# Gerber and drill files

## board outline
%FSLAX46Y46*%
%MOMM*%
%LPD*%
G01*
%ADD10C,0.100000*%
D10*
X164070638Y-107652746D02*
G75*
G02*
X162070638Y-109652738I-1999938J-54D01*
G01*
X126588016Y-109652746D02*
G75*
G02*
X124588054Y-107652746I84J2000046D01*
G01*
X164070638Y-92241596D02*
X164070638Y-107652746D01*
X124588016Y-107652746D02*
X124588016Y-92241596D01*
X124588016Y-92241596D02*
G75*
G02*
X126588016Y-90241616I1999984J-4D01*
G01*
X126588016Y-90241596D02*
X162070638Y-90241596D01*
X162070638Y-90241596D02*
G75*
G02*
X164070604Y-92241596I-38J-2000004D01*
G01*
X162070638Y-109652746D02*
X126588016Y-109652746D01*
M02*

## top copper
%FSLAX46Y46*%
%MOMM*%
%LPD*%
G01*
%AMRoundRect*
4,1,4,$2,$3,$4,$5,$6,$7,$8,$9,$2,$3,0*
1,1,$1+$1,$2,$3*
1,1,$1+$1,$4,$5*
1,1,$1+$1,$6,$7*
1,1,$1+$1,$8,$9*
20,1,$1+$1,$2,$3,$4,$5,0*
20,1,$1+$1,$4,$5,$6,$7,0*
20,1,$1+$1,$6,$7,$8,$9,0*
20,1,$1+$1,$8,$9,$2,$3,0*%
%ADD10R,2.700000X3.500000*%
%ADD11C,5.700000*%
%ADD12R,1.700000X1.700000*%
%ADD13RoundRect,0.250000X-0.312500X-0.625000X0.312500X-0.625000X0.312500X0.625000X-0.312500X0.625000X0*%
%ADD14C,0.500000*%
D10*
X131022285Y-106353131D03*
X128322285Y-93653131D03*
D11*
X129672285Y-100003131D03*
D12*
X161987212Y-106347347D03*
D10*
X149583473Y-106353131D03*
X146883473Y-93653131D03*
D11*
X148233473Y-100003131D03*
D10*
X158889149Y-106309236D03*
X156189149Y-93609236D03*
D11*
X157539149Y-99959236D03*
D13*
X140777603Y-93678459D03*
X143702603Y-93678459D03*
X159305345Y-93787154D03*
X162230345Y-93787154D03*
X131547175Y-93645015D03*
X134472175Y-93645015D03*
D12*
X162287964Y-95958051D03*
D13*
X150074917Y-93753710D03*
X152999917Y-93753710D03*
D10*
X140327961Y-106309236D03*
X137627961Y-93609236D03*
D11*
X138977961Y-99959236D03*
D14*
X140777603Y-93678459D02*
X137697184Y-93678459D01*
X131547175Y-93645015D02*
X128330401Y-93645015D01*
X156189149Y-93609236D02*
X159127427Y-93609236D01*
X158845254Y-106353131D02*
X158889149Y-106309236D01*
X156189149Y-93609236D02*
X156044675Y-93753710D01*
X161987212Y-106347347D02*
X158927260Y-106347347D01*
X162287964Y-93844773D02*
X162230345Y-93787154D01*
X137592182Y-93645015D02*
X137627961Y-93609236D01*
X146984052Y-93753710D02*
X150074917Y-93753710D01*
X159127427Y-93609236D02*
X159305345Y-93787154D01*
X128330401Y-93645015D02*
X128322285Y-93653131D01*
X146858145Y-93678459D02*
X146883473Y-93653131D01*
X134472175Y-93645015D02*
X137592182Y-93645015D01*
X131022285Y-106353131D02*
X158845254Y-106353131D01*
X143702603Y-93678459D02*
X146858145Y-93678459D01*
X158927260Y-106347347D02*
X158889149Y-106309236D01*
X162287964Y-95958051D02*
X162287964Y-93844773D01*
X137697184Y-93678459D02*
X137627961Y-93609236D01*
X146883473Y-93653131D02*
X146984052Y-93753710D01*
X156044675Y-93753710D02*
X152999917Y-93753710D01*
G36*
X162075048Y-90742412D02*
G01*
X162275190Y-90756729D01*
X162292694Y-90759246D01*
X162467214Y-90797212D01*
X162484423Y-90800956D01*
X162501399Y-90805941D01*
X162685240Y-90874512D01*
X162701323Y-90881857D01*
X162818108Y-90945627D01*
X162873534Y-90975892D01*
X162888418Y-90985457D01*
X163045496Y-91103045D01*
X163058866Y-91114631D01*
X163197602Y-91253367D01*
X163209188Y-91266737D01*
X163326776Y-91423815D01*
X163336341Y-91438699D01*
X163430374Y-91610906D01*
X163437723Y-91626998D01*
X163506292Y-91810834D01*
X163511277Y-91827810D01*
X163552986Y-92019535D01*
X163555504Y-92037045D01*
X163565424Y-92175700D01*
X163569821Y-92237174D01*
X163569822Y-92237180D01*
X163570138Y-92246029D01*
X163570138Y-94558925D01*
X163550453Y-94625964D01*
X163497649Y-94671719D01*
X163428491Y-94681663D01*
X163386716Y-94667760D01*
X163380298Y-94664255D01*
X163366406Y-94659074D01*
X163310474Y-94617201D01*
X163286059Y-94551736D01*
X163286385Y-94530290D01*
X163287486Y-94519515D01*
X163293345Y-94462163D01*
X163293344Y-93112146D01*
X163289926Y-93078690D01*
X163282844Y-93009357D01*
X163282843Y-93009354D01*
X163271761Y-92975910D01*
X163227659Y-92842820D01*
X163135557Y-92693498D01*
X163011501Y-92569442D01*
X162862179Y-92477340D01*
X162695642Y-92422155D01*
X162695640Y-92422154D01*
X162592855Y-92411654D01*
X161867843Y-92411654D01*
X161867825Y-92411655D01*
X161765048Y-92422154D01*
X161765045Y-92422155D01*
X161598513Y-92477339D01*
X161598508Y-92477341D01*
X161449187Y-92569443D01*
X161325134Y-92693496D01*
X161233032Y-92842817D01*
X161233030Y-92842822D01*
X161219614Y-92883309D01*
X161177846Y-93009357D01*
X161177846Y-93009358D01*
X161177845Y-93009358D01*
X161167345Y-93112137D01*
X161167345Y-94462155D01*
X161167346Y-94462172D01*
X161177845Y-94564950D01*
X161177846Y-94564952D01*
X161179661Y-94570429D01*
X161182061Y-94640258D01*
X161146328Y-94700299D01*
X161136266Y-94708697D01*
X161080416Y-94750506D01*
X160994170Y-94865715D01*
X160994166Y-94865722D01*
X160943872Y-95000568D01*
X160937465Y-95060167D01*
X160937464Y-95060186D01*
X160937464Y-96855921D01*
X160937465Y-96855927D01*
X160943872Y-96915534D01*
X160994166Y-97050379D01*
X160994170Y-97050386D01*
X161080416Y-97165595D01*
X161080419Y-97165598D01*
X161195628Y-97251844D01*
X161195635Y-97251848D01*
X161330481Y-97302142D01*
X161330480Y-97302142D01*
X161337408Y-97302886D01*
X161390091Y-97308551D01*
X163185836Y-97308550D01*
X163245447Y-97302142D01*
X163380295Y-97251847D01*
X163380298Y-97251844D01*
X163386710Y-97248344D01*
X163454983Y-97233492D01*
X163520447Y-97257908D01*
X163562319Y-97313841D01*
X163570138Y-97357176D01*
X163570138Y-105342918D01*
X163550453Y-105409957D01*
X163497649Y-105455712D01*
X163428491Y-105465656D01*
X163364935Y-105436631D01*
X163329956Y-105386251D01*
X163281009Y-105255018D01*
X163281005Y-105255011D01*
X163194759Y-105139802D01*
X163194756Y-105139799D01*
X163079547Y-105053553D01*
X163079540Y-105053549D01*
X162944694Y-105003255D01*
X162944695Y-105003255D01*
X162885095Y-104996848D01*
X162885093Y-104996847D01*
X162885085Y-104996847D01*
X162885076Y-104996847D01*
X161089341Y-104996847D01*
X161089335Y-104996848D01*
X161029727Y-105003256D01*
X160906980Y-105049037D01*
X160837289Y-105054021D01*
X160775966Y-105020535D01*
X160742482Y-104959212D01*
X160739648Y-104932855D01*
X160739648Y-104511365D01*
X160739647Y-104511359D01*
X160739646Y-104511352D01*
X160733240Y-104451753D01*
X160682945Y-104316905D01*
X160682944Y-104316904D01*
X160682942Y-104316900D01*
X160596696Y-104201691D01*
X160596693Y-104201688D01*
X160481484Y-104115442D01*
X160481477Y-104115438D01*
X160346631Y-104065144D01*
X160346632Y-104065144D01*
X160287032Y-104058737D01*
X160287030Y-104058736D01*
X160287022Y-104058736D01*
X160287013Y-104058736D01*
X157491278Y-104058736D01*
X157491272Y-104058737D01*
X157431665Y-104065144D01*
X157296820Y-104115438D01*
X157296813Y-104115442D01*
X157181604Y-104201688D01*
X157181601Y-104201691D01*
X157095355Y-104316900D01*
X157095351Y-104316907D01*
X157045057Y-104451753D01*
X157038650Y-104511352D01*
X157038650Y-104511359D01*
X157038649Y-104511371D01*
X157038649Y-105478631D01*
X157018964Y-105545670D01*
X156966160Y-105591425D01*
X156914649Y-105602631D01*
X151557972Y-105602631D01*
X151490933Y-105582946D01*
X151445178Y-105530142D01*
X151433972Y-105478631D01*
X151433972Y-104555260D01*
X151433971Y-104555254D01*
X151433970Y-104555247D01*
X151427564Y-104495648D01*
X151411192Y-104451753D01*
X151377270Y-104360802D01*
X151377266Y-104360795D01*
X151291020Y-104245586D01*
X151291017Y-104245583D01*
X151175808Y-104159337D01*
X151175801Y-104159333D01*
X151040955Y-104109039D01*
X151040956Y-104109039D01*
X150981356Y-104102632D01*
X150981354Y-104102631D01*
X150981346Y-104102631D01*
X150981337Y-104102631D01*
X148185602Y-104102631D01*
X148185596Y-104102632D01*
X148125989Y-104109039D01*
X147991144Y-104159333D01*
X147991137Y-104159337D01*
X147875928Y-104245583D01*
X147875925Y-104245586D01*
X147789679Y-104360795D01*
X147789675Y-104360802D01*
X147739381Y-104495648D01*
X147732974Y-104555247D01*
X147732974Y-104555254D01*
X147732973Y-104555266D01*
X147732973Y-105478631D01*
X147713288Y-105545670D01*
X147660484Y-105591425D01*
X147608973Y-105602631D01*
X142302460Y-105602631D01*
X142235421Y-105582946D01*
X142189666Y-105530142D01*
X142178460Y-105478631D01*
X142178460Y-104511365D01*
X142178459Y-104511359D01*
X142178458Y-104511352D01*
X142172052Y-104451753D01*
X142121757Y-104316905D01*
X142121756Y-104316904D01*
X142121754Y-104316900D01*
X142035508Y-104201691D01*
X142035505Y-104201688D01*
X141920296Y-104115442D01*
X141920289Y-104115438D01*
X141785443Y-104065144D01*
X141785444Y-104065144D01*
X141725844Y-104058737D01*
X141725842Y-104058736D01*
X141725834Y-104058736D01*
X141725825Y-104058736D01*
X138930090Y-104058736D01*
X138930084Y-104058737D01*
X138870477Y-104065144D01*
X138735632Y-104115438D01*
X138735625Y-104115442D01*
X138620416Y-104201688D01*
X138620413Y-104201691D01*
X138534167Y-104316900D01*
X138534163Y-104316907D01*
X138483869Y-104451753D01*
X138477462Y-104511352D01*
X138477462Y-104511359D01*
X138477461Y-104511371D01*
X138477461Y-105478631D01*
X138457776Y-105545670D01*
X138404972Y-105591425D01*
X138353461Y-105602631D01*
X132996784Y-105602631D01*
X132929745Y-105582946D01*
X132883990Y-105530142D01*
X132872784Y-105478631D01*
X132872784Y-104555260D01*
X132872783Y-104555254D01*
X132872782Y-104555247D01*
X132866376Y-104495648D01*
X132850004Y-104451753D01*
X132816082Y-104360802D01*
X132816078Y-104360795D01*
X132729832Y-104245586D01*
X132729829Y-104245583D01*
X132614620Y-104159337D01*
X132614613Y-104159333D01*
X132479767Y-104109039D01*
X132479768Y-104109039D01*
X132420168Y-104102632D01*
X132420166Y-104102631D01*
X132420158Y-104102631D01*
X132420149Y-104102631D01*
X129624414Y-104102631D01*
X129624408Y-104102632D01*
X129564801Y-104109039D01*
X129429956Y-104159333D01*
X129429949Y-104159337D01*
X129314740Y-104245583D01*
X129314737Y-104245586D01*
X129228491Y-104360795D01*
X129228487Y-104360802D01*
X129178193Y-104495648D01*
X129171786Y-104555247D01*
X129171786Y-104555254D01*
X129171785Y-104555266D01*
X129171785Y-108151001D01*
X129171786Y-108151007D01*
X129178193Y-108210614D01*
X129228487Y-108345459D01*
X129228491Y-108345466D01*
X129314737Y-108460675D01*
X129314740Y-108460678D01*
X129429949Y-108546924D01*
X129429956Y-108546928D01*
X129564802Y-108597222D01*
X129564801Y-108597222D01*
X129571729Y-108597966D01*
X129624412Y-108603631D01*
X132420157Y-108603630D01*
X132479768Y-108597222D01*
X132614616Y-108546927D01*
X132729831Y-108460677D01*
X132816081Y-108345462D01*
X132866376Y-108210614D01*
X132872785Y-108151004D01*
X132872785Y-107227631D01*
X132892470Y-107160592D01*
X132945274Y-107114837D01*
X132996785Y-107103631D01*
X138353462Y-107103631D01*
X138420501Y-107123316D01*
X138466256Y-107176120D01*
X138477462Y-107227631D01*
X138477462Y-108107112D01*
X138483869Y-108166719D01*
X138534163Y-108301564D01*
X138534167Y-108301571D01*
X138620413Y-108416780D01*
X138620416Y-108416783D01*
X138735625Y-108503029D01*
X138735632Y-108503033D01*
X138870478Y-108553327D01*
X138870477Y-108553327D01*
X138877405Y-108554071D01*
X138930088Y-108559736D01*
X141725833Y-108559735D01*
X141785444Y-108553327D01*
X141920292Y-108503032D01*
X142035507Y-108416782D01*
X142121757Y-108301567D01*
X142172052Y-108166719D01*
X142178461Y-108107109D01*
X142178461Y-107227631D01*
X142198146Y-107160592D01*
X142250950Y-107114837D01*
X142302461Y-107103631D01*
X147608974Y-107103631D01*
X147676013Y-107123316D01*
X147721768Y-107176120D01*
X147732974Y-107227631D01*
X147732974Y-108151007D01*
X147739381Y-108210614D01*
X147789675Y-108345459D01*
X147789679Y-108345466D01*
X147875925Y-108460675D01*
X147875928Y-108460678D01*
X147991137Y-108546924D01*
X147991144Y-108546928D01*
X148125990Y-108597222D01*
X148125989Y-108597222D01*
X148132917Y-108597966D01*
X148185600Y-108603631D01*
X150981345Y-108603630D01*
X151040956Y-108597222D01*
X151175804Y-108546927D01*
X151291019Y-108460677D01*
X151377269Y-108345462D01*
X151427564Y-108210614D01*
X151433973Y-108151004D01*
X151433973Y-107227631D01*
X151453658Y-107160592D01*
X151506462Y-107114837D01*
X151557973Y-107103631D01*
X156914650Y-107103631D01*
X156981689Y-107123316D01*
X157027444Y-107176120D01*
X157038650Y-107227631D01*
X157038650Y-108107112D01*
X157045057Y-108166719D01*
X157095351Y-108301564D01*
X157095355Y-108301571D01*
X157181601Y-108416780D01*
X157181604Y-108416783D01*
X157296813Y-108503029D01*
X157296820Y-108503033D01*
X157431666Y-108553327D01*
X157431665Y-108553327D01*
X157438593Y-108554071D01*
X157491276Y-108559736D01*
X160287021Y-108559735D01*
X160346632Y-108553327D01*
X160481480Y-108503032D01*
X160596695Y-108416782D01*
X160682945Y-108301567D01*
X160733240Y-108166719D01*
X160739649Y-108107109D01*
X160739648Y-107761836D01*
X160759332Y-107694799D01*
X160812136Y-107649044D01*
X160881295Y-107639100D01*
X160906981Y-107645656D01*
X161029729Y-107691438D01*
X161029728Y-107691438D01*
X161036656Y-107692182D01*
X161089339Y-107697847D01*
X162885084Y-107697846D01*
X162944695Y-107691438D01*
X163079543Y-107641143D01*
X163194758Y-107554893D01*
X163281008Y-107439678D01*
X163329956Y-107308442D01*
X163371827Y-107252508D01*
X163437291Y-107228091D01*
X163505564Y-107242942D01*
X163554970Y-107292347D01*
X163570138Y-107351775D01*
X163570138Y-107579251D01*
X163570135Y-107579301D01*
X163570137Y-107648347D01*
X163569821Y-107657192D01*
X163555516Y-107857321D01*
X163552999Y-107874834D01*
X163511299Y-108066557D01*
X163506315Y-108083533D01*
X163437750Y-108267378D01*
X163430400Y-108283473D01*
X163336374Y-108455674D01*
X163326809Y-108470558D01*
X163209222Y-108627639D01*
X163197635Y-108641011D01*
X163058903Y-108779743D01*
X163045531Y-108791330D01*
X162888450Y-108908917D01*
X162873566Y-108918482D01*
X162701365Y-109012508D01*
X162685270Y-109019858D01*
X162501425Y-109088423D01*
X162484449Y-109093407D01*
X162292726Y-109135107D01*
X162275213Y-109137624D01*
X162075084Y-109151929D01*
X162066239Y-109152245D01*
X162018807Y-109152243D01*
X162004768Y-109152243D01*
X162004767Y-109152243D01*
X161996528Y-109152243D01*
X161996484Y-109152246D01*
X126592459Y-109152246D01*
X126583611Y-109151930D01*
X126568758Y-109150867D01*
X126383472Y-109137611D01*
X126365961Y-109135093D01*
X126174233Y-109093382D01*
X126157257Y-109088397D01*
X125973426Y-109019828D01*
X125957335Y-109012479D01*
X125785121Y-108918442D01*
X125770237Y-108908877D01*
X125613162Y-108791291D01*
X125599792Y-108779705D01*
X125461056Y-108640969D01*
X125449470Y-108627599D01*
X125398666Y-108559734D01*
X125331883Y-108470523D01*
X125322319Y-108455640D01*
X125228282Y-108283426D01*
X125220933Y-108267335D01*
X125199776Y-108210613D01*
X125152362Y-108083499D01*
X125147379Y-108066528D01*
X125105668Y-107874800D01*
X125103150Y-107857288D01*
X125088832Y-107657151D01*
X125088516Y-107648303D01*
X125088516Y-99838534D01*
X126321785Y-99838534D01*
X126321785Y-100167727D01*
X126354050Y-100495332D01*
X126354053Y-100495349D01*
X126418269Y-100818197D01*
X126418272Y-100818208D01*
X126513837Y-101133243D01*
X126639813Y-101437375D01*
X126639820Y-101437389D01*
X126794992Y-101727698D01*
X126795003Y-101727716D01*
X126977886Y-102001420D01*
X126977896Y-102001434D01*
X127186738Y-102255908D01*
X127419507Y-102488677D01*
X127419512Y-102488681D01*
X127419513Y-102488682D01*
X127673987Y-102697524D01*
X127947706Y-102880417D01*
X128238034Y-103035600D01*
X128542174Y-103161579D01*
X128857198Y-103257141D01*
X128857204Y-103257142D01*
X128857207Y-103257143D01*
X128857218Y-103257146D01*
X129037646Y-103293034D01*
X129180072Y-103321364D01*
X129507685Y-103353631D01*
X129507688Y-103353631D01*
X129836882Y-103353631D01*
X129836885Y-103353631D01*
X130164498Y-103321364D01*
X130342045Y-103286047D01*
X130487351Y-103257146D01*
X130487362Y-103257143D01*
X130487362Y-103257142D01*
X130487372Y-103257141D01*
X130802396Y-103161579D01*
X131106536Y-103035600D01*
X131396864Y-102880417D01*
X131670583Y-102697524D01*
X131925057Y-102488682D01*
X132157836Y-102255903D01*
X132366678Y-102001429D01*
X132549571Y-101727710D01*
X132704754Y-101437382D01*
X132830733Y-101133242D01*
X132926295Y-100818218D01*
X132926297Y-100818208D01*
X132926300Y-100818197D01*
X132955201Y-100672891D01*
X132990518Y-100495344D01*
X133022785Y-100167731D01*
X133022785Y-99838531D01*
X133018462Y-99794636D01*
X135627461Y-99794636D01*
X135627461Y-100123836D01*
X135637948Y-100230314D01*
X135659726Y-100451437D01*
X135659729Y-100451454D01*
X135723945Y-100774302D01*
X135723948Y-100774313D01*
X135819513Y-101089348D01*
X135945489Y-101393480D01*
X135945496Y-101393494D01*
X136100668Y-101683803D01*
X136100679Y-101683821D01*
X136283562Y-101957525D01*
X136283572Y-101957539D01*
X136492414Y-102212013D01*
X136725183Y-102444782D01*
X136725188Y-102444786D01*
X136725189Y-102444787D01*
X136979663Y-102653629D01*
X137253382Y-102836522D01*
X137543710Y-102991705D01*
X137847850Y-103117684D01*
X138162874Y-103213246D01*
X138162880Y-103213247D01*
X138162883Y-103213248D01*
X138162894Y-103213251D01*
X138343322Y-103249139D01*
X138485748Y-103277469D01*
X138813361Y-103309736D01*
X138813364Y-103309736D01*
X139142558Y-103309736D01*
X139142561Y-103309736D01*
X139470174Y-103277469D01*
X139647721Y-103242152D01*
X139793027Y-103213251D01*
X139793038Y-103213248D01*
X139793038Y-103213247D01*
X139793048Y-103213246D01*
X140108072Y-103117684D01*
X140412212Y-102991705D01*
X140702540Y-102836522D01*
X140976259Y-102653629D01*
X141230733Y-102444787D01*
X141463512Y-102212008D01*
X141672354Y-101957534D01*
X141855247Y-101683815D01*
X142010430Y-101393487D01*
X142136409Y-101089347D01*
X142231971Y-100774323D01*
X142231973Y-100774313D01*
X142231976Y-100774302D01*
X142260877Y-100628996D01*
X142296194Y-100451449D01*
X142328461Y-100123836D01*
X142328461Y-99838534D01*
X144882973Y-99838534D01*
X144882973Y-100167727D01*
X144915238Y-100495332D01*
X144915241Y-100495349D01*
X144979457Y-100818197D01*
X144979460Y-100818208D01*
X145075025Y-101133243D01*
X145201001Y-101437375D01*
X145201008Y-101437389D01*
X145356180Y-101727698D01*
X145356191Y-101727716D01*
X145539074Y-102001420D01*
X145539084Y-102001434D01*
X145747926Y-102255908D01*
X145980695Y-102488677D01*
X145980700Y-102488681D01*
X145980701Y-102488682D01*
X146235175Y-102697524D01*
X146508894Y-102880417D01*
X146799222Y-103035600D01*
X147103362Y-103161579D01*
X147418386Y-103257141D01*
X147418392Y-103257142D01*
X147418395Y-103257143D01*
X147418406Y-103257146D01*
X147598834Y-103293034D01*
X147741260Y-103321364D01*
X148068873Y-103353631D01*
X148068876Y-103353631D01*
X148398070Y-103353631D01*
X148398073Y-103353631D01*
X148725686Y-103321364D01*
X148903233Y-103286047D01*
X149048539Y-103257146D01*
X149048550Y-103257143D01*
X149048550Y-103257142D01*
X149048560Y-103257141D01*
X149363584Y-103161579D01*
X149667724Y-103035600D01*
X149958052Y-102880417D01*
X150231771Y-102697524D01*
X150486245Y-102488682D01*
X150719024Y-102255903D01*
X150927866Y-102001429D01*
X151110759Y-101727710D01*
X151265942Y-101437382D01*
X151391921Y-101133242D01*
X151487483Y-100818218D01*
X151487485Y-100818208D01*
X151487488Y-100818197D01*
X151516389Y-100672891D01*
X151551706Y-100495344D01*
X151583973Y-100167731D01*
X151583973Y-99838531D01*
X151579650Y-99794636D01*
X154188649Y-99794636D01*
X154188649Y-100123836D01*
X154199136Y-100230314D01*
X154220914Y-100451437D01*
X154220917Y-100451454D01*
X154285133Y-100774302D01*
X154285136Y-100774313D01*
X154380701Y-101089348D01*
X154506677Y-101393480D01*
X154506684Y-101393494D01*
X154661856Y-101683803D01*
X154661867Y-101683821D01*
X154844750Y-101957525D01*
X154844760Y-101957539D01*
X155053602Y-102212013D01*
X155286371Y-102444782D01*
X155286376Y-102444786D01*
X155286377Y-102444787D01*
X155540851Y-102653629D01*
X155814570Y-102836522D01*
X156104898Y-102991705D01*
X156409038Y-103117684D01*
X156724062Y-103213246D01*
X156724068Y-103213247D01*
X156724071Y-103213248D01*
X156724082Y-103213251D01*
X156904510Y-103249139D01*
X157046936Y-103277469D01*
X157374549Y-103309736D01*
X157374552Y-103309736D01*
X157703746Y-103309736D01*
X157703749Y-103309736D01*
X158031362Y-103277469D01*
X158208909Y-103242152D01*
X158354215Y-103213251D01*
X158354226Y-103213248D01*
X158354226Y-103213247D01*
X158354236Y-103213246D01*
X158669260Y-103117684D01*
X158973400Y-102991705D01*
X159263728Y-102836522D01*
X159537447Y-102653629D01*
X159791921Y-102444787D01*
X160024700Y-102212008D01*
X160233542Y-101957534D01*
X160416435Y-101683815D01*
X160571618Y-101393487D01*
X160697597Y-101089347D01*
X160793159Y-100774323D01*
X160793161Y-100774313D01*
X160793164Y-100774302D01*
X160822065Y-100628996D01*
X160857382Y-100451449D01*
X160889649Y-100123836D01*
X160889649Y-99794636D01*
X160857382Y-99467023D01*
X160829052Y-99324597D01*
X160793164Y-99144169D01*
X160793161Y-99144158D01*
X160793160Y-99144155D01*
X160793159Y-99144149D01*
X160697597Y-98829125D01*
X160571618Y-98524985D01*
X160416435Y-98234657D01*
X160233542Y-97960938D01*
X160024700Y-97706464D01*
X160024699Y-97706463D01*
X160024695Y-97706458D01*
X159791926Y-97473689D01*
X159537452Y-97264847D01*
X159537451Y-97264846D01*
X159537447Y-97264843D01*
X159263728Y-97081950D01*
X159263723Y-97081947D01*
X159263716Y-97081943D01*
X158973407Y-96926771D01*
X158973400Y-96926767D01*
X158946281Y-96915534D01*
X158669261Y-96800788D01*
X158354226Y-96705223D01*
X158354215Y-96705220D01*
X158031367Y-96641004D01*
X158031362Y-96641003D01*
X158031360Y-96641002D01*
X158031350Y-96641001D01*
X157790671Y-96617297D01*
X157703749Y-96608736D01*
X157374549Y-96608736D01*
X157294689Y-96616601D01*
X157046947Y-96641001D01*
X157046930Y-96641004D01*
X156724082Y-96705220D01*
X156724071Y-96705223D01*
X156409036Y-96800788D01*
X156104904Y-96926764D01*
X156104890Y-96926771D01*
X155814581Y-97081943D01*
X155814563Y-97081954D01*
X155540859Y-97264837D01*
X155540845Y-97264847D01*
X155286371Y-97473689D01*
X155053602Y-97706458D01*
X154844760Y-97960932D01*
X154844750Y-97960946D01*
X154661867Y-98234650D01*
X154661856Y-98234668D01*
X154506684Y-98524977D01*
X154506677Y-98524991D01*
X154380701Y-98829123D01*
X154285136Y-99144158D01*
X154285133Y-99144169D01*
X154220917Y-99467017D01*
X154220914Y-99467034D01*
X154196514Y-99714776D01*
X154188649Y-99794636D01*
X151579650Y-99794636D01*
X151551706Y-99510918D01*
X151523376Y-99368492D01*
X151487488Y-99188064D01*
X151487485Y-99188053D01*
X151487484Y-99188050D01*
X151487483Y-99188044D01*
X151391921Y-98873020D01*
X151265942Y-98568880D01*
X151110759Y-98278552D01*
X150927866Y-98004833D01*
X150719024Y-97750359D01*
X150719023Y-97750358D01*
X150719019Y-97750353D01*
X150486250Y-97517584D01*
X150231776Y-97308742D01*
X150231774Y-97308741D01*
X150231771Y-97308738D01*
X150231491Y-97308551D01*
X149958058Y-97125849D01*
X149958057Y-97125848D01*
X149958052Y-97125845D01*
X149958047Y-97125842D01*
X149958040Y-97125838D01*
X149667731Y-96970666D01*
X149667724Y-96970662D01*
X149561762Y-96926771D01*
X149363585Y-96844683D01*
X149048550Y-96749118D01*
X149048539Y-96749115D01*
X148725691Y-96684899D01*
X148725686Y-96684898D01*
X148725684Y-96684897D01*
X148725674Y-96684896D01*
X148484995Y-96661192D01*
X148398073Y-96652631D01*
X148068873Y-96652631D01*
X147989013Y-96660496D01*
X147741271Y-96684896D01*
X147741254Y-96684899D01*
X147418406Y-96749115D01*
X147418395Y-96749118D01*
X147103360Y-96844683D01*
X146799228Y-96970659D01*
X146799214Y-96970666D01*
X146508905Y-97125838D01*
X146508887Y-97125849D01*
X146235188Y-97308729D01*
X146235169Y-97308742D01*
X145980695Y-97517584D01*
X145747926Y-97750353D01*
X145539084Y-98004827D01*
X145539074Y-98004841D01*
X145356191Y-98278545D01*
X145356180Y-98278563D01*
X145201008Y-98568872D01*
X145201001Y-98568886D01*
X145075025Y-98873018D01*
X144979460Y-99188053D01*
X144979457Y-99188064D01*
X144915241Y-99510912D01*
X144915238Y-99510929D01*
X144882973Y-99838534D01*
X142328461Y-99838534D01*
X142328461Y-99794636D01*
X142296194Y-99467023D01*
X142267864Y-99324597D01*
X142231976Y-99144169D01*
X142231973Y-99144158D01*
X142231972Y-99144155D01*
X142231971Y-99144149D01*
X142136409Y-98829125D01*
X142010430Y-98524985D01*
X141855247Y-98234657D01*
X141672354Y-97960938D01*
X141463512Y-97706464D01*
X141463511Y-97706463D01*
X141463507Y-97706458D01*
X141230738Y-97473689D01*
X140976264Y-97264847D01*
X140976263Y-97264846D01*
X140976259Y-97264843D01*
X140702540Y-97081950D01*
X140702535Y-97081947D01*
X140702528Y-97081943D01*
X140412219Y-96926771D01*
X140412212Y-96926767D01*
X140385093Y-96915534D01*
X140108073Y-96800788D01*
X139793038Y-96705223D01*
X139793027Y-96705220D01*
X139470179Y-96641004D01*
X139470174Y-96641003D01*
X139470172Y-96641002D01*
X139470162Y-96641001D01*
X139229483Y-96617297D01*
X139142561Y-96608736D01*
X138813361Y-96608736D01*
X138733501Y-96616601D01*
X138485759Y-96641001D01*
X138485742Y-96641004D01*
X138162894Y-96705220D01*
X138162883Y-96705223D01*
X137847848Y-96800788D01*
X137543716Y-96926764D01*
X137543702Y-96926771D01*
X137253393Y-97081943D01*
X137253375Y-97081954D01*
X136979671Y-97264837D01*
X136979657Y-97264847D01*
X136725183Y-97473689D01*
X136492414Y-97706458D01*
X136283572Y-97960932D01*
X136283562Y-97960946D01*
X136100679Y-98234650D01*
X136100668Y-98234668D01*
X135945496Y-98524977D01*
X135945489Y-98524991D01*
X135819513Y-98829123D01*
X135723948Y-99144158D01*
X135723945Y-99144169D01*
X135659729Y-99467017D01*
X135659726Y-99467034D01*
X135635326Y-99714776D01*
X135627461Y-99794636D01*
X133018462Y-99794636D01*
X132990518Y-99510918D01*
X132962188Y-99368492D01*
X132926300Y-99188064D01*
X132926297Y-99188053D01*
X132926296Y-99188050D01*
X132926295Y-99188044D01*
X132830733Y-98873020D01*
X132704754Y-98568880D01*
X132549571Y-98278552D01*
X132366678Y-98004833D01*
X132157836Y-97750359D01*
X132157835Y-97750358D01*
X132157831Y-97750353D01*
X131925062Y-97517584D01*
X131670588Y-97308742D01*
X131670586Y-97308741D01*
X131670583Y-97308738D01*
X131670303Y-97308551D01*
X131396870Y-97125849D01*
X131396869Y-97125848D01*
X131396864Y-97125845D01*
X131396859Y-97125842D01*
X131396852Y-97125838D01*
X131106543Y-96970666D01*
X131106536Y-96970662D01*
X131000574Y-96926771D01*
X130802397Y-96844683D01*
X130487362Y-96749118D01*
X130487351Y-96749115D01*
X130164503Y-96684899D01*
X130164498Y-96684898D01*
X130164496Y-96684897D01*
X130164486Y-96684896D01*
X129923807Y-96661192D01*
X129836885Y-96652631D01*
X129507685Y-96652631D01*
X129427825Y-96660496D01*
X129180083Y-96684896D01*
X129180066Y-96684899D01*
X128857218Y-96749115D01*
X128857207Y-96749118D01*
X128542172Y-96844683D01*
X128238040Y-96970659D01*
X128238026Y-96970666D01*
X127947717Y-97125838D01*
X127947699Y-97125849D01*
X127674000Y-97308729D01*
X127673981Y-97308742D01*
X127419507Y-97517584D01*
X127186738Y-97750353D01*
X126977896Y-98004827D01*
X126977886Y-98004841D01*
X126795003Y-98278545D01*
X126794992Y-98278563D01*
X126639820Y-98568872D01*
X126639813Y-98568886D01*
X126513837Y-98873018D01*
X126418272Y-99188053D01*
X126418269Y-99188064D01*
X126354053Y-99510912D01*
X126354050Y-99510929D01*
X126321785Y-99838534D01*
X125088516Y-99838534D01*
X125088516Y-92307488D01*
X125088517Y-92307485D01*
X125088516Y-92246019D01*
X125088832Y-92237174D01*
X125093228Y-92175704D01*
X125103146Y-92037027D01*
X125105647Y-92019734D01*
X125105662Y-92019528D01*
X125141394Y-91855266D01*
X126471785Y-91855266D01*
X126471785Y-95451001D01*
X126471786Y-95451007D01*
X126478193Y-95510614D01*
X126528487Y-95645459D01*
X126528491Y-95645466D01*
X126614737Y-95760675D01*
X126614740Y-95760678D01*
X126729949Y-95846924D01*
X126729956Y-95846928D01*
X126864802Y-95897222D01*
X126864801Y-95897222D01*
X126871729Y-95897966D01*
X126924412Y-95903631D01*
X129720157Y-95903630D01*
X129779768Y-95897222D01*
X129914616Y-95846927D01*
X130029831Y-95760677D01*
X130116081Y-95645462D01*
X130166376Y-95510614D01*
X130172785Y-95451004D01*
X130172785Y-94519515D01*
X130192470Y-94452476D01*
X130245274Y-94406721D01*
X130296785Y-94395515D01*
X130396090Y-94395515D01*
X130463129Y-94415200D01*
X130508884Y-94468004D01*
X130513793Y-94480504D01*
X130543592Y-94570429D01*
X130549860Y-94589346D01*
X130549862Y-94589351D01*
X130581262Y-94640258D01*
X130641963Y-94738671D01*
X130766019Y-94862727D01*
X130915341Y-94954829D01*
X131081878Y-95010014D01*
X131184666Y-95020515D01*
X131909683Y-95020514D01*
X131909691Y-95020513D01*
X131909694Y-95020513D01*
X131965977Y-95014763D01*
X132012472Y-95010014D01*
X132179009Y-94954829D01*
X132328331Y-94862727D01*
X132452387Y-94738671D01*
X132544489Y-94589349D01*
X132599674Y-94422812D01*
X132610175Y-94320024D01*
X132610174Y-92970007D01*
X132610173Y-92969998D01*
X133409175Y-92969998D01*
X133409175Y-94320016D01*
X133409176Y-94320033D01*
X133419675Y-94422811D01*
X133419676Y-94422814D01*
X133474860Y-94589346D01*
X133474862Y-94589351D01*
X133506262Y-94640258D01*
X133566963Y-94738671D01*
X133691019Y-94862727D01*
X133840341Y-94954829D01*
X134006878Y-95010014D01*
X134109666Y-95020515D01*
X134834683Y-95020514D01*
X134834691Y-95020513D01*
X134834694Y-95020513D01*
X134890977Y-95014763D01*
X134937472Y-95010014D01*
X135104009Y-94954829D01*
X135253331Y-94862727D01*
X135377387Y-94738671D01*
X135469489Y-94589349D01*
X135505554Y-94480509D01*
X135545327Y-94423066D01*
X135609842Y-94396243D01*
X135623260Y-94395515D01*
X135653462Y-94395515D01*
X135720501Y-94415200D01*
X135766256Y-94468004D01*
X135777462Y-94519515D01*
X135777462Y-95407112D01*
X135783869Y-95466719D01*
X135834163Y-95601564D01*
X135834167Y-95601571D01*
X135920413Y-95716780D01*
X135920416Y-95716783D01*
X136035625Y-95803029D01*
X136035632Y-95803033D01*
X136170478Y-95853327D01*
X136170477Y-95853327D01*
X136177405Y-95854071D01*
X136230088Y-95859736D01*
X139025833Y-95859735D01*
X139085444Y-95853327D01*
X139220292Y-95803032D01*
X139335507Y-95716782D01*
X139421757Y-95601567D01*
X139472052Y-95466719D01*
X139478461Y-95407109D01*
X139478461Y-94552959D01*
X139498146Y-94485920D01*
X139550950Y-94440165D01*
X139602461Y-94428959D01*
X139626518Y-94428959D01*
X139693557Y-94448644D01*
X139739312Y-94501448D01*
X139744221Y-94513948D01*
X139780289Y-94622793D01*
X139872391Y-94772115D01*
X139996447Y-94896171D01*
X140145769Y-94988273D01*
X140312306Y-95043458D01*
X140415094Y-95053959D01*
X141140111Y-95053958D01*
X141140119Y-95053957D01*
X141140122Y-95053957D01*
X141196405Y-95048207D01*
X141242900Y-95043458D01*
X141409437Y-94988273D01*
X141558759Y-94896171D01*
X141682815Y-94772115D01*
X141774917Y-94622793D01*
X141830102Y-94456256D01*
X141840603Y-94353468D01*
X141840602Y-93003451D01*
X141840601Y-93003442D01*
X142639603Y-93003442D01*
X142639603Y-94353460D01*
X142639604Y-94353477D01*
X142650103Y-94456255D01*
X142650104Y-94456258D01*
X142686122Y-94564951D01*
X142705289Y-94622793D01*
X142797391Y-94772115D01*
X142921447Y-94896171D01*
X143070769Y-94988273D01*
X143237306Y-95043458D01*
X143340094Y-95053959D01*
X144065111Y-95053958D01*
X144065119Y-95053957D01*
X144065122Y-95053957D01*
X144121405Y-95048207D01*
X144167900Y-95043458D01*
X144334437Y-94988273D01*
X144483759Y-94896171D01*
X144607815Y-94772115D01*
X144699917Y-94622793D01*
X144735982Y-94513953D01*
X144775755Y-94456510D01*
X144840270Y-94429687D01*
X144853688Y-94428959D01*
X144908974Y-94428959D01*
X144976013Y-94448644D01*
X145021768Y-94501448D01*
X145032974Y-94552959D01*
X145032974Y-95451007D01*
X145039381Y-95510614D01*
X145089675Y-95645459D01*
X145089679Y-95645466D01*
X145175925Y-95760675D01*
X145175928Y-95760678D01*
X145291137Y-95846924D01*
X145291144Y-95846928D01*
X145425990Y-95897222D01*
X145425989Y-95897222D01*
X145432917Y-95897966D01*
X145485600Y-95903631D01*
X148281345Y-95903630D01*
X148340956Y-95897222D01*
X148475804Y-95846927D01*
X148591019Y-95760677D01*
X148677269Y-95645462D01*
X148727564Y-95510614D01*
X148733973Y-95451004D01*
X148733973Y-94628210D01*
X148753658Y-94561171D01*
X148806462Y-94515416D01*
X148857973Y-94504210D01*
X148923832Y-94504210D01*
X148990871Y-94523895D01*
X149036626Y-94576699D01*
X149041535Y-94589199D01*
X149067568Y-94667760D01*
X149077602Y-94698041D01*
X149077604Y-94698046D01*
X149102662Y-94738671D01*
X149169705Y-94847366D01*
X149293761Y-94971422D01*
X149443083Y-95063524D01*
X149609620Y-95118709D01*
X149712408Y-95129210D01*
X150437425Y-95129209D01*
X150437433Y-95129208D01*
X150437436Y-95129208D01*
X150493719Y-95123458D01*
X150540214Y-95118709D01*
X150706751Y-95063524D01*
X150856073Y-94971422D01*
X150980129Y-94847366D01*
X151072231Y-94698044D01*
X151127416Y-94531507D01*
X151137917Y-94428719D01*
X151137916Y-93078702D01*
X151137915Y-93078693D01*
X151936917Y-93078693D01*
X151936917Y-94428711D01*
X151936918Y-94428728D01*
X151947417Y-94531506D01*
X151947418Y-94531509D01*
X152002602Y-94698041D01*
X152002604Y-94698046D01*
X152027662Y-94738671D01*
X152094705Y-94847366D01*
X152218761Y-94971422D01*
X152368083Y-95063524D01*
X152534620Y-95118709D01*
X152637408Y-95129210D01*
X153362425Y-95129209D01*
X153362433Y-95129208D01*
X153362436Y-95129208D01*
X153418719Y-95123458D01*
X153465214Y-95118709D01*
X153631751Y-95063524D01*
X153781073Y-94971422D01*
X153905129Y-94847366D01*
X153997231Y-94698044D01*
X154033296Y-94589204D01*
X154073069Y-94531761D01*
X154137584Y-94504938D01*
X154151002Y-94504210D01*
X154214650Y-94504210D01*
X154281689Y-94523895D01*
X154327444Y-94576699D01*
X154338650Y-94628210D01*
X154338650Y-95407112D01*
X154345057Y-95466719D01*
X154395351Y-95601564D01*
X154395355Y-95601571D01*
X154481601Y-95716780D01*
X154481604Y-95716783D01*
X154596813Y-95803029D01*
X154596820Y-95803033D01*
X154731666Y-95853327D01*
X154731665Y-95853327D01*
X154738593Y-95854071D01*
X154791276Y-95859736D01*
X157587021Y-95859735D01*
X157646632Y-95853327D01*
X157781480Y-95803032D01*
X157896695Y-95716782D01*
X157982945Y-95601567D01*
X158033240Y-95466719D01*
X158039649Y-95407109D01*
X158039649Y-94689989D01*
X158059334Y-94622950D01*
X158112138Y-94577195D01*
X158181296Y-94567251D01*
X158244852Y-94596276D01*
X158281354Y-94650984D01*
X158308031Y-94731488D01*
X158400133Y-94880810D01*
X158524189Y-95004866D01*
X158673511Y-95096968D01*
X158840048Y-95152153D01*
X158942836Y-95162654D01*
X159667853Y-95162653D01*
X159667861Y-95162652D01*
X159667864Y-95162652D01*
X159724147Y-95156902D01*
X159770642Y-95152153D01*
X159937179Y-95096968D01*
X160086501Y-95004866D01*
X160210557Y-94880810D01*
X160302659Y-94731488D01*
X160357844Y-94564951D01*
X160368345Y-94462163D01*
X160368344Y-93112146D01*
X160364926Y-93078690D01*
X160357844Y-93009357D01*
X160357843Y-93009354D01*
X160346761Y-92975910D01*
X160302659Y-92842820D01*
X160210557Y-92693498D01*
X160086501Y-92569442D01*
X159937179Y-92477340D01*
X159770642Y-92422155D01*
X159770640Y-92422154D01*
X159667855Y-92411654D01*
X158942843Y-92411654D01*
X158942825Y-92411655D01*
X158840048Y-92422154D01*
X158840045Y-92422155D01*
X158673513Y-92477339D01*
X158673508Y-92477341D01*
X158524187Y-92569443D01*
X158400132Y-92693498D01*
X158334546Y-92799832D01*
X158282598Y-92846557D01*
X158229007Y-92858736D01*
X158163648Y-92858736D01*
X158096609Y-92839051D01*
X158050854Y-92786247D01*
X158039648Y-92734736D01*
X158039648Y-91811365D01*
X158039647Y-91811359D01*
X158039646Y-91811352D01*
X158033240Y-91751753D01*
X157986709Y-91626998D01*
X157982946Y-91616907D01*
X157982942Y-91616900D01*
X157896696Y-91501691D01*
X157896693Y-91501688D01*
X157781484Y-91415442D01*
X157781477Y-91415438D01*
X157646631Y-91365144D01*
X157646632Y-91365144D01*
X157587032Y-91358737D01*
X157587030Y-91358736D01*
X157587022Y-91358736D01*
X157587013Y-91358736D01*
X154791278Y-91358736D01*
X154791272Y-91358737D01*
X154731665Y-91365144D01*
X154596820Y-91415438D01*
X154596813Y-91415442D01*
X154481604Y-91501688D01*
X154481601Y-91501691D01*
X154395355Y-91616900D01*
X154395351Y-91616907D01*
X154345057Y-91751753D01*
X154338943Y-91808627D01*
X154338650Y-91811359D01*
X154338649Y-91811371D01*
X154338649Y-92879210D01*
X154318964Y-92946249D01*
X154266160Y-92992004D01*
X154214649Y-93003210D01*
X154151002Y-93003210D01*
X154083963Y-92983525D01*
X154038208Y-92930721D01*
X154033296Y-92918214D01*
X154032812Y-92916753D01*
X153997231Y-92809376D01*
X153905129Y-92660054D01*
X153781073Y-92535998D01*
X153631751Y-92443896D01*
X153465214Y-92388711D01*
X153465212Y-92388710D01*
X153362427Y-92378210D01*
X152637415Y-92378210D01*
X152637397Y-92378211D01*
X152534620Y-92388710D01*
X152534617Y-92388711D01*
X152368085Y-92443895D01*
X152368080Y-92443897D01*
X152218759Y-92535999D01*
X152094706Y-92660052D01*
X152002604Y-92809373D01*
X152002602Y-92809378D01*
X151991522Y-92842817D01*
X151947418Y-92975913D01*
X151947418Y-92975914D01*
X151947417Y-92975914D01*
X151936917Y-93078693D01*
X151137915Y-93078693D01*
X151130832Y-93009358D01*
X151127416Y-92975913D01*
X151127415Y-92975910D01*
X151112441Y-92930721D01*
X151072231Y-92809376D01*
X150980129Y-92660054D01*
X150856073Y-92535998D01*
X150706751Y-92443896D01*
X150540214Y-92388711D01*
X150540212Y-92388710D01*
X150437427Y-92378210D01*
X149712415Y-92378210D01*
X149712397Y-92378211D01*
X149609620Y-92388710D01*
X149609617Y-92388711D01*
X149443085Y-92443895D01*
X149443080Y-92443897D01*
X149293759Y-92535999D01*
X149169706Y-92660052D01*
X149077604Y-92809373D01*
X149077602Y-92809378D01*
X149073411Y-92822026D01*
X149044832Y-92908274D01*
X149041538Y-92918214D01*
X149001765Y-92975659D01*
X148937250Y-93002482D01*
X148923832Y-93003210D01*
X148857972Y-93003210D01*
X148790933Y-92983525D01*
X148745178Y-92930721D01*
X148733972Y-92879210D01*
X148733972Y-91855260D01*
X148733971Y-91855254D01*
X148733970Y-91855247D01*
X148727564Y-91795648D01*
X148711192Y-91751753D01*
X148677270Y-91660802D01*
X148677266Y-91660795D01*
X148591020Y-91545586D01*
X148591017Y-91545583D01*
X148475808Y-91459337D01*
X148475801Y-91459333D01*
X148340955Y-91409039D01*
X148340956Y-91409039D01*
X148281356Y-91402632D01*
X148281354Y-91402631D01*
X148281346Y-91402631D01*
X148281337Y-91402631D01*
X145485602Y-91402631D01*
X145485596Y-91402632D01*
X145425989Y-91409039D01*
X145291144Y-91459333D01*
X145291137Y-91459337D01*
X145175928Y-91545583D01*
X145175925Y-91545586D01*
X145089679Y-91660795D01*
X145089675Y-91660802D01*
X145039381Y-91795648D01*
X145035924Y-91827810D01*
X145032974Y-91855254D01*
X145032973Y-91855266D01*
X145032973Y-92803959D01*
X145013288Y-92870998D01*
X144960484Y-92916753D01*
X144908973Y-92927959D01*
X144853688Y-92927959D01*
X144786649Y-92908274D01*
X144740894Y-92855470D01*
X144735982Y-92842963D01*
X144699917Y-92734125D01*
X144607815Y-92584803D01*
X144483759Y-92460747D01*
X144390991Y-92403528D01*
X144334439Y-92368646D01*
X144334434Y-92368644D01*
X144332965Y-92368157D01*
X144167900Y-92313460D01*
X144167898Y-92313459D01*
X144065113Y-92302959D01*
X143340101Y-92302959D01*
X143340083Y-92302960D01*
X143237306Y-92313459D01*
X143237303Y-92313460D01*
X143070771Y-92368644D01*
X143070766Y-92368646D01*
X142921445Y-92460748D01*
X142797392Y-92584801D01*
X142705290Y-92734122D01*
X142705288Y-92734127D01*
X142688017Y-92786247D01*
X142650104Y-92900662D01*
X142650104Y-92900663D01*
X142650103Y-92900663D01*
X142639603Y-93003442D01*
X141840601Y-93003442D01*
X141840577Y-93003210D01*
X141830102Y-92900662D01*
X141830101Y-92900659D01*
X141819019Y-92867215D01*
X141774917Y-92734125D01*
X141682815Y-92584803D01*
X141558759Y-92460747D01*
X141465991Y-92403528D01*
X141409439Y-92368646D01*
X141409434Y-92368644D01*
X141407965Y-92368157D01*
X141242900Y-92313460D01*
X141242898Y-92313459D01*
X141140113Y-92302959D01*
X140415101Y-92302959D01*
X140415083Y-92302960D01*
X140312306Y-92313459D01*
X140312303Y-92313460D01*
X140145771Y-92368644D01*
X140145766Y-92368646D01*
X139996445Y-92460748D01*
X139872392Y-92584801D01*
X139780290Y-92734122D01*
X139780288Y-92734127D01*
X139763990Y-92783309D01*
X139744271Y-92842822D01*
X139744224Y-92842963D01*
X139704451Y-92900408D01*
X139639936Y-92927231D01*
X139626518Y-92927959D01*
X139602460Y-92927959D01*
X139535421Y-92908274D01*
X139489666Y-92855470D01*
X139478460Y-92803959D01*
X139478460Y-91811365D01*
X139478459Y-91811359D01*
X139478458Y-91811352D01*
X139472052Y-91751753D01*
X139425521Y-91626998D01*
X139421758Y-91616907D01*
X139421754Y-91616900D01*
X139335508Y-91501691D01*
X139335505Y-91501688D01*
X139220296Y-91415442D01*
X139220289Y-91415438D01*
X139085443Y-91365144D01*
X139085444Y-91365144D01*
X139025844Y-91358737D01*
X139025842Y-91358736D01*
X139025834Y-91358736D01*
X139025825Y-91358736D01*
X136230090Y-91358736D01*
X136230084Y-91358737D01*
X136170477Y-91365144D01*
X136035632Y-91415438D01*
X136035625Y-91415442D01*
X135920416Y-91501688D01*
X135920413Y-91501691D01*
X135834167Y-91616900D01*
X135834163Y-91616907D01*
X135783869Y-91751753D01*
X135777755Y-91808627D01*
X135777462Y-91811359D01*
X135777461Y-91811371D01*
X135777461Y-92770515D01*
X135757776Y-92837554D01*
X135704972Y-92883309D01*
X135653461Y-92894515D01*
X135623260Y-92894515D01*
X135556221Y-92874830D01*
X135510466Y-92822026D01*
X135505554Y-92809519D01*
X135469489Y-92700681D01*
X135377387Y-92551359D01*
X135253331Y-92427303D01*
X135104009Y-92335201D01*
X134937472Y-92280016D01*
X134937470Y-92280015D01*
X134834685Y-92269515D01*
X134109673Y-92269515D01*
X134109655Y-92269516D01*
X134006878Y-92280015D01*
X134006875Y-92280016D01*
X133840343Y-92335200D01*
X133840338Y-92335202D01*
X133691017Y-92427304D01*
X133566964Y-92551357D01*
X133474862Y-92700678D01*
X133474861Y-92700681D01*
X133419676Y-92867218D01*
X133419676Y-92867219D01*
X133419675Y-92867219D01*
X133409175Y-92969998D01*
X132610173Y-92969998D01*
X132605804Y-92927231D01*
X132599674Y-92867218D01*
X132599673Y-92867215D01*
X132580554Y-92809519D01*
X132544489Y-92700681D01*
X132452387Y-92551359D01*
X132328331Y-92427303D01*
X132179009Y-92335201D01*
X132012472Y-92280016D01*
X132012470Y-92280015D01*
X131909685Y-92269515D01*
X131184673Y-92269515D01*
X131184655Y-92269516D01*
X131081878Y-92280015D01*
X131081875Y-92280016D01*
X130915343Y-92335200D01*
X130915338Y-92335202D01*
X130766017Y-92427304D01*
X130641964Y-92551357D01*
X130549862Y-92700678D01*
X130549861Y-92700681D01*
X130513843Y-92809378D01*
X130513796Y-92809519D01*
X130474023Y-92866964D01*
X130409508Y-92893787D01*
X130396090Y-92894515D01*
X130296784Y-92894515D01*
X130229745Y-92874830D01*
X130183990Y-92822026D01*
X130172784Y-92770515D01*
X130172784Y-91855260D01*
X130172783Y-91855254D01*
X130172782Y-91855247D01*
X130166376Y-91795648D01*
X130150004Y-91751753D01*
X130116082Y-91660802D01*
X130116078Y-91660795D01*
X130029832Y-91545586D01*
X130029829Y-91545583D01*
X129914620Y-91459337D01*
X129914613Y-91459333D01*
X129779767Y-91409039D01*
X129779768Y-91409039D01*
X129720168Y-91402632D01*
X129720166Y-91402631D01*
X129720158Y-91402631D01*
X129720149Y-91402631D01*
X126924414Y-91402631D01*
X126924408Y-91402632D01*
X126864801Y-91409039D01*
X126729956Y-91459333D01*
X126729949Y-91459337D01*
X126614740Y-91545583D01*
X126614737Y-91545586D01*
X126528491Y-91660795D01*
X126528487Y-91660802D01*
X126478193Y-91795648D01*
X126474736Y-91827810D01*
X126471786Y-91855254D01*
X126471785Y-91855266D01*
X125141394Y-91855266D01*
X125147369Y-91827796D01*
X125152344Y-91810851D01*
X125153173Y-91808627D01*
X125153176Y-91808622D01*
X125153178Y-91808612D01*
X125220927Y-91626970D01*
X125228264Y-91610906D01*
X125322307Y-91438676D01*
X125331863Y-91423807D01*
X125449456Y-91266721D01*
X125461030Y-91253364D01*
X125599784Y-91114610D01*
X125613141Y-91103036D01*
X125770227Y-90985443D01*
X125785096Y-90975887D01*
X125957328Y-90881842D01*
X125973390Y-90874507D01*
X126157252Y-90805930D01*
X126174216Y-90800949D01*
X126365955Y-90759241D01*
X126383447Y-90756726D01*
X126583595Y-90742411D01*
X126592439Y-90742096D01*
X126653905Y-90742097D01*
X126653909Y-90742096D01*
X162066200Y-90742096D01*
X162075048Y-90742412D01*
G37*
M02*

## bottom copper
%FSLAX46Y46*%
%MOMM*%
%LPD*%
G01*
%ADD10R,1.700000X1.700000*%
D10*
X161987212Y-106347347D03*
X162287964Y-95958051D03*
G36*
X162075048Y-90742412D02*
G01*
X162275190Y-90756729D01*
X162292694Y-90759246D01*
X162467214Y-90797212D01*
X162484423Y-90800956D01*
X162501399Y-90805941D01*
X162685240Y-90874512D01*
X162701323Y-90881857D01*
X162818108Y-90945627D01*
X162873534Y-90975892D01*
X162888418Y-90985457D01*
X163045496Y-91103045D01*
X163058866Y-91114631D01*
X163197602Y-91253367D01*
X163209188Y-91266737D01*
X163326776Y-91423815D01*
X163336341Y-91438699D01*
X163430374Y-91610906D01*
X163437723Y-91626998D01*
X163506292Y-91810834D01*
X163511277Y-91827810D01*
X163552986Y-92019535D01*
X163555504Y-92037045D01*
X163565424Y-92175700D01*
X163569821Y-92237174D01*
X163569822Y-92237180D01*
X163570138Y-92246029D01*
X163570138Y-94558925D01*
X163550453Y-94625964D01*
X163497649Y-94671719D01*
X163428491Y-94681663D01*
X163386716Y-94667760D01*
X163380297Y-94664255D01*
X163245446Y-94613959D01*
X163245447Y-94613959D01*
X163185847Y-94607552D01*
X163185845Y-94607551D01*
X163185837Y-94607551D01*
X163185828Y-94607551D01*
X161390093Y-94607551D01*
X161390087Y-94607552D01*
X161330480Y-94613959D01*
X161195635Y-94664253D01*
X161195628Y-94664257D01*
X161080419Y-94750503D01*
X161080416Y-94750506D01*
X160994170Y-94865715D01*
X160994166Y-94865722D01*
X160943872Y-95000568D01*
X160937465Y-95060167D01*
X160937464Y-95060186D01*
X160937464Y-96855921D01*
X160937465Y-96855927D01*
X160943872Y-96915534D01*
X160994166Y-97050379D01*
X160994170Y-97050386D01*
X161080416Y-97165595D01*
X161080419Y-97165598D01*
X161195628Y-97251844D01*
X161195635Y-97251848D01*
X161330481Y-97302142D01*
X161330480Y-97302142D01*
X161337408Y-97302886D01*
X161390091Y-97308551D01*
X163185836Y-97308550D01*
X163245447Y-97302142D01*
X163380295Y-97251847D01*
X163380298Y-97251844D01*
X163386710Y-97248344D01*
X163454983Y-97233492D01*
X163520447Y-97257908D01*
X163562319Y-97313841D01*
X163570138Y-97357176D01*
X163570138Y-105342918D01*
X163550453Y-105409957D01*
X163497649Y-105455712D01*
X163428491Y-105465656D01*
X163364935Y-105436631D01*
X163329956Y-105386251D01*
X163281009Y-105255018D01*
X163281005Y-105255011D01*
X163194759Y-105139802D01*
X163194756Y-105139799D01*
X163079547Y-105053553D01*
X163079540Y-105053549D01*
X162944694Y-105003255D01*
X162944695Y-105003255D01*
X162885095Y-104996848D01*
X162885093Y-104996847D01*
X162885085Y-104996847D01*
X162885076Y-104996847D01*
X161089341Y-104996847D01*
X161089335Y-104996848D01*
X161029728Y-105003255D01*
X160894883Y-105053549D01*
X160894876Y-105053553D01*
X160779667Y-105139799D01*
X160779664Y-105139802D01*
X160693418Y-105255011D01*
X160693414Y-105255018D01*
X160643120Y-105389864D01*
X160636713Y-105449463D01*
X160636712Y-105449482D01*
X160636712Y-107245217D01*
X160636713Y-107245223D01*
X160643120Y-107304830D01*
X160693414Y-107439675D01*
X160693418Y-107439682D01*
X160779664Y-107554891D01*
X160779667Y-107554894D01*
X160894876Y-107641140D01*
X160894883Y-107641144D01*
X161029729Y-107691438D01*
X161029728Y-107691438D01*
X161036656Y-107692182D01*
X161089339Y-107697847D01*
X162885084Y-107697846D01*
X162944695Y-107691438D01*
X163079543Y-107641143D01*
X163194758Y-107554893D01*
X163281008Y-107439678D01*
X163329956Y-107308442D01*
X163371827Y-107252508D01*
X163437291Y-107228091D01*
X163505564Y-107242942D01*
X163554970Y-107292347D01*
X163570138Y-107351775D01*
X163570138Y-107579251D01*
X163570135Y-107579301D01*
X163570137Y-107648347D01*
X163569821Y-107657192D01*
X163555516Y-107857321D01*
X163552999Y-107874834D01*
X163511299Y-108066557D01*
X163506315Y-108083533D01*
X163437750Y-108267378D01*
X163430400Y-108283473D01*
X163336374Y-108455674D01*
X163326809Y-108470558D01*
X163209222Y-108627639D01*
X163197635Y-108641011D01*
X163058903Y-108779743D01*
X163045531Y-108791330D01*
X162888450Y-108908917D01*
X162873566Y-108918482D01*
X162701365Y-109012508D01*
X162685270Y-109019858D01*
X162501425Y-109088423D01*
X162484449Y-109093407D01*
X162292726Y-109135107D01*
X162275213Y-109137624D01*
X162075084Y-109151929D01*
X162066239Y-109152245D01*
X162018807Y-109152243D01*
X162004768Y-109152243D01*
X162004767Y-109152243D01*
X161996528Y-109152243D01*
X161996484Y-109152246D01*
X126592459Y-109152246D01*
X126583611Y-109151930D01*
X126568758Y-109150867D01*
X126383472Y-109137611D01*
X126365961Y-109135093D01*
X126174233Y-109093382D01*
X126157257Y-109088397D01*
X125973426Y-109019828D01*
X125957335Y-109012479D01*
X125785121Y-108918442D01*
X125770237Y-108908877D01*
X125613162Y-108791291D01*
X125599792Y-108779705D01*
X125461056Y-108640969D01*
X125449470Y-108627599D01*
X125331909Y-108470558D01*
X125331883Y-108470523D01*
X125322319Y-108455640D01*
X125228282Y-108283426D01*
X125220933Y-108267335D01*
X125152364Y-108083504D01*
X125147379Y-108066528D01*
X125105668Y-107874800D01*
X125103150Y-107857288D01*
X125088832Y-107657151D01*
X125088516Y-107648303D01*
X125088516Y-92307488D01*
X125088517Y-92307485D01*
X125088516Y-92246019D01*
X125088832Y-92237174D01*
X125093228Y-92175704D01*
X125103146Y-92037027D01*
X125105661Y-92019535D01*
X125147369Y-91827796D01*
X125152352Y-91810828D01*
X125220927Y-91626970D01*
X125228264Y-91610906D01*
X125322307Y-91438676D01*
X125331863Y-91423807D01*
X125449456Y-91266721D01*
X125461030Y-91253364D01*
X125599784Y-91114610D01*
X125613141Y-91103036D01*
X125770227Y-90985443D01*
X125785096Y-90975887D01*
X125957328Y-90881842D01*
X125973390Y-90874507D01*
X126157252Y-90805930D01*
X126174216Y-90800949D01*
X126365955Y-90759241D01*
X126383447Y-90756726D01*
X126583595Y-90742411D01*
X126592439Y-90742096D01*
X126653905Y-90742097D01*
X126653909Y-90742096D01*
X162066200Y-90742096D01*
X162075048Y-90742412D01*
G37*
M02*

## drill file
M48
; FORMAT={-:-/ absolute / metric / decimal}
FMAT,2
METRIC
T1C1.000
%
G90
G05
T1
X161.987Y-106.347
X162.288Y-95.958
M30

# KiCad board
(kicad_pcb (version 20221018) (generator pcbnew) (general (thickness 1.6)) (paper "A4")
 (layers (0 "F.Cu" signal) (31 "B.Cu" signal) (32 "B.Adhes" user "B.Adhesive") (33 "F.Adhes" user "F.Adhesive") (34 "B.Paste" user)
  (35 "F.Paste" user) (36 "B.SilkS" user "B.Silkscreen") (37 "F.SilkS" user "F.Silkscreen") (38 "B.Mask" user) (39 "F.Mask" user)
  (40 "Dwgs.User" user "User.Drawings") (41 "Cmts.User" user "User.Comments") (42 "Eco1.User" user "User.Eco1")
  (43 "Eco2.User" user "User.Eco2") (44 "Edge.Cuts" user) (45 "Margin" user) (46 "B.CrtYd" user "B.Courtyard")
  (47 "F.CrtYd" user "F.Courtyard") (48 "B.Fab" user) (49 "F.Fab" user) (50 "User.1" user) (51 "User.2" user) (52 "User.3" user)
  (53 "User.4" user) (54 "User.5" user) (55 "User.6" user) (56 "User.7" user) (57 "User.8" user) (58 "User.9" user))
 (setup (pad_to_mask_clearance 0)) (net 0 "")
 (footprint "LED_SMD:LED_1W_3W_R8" (layer "F.Cu") (at 129.672285 100.003131 90)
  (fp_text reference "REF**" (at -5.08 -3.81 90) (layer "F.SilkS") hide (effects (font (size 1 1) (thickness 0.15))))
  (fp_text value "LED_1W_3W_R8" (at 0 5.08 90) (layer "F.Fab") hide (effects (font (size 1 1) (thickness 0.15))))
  (pad "1" smd rect (at -6.35 1.35 90) (size 3.5 2.7) (layers "F.Cu" "F.Paste" "F.Mask"))
  (pad "2" smd rect (at 6.35 -1.35 90) (size 3.5 2.7) (layers "F.Cu" "F.Paste" "F.Mask"))
  (pad "3" smd circle (at 0 0 90) (size 5.7 5.7) (layers "F.Cu" "F.Paste" "F.Mask")))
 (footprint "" (layer "F.Cu") (at 161.987212 106.347347)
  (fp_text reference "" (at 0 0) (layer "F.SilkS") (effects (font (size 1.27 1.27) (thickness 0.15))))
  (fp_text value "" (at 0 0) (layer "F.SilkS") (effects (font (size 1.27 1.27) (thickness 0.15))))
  (pad "1" thru_hole rect (at 0 0 180) (size 1.7 1.7) (drill 1) (layers "*.Cu" "*.Mask")))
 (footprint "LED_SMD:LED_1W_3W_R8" (layer "F.Cu") (at 148.233473 100.003131 90)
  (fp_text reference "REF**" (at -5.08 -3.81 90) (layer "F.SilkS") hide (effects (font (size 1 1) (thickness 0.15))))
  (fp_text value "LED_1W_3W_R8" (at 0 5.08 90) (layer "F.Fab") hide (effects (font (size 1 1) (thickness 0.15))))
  (pad "1" smd rect (at -6.35 1.35 90) (size 3.5 2.7) (layers "F.Cu" "F.Paste" "F.Mask"))
  (pad "2" smd rect (at 6.35 -1.35 90) (size 3.5 2.7) (layers "F.Cu" "F.Paste" "F.Mask"))
  (pad "3" smd circle (at 0 0 90) (size 5.7 5.7) (layers "F.Cu" "F.Paste" "F.Mask")))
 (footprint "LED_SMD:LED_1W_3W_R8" (layer "F.Cu") (at 157.539149 99.959236 90)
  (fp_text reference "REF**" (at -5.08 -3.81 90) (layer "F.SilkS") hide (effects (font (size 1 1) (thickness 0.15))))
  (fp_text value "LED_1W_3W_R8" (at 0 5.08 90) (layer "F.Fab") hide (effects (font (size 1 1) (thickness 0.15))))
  (pad "1" smd rect (at -6.35 1.35 90) (size 3.5 2.7) (layers "F.Cu" "F.Paste" "F.Mask"))
  (pad "2" smd rect (at 6.35 -1.35 90) (size 3.5 2.7) (layers "F.Cu" "F.Paste" "F.Mask"))
  (pad "3" smd circle (at 0 0 90) (size 5.7 5.7) (layers "F.Cu" "F.Paste" "F.Mask")))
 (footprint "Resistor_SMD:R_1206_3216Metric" (layer "F.Cu") (at 142.240103 93.678459)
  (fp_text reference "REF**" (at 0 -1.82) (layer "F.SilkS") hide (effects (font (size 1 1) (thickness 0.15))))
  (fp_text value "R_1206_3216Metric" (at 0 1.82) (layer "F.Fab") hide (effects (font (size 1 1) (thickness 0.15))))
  (pad "1" smd roundrect (at -1.4625 0) (size 1.125 1.75) (layers "F.Cu" "F.Paste" "F.Mask") (roundrect_rratio 0.222222))
  (pad "2" smd roundrect (at 1.4625 0) (size 1.125 1.75) (layers "F.Cu" "F.Paste" "F.Mask") (roundrect_rratio 0.222222)))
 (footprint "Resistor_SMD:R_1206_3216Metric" (layer "F.Cu") (at 160.767845 93.787154)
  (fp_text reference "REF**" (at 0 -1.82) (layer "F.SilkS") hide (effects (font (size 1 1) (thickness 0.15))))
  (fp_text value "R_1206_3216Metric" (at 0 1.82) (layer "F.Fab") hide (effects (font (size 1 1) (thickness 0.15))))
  (pad "1" smd roundrect (at -1.4625 0) (size 1.125 1.75) (layers "F.Cu" "F.Paste" "F.Mask") (roundrect_rratio 0.222222))
  (pad "2" smd roundrect (at 1.4625 0) (size 1.125 1.75) (layers "F.Cu" "F.Paste" "F.Mask") (roundrect_rratio 0.222222)))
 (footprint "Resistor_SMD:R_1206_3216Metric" (layer "F.Cu") (at 133.009675 93.645015)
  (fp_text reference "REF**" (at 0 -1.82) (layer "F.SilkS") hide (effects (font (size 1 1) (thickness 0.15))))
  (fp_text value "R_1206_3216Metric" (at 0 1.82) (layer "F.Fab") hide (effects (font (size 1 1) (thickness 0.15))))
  (pad "1" smd roundrect (at -1.4625 0) (size 1.125 1.75) (layers "F.Cu" "F.Paste" "F.Mask") (roundrect_rratio 0.222222))
  (pad "2" smd roundrect (at 1.4625 0) (size 1.125 1.75) (layers "F.Cu" "F.Paste" "F.Mask") (roundrect_rratio 0.222222)))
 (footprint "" (layer "F.Cu") (at 162.287964 95.958051)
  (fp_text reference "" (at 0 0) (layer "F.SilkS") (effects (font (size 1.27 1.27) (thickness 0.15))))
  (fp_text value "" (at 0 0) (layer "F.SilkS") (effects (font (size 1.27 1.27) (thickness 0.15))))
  (pad "1" thru_hole rect (at 0 0 180) (size 1.7 1.7) (drill 1) (layers "*.Cu" "*.Mask")))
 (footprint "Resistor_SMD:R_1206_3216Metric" (layer "F.Cu") (at 151.537417 93.75371)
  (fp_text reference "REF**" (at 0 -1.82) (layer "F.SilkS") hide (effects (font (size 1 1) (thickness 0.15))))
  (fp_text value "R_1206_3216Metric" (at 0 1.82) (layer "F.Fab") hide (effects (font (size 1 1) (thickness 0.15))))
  (pad "1" smd roundrect (at -1.4625 0) (size 1.125 1.75) (layers "F.Cu" "F.Paste" "F.Mask") (roundrect_rratio 0.222222))
  (pad "2" smd roundrect (at 1.4625 0) (size 1.125 1.75) (layers "F.Cu" "F.Paste" "F.Mask") (roundrect_rratio 0.222222)))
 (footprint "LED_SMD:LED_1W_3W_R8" (layer "F.Cu") (at 138.977961 99.959236 90)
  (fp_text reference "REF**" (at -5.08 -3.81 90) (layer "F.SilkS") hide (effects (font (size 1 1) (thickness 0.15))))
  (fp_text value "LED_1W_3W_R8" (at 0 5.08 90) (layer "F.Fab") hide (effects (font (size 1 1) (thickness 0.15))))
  (pad "1" smd rect (at -6.35 1.35 90) (size 3.5 2.7) (layers "F.Cu" "F.Paste" "F.Mask"))
  (pad "2" smd rect (at 6.35 -1.35 90) (size 3.5 2.7) (layers "F.Cu" "F.Paste" "F.Mask"))
  (pad "3" smd circle (at 0 0 90) (size 5.7 5.7) (layers "F.Cu" "F.Paste" "F.Mask")))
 (gr_arc (start 164.070638 107.652746) (mid 163.484878 109.066986) (end 162.070638 109.652746) (stroke (width 0.1) (type default))
  (layer "Edge.Cuts"))
 (gr_arc (start 126.588016 109.652746) (mid 125.173816 109.066946) (end 124.588016 107.652746) (stroke (width 0.1) (type default))
  (layer "Edge.Cuts"))
 (gr_line (start 164.070638 92.241596) (end 164.070638 107.652746) (stroke (width 0.1) (type default)) (layer "Edge.Cuts"))
 (gr_line (start 124.588016 107.652746) (end 124.588016 92.241596) (stroke (width 0.1) (type default)) (layer "Edge.Cuts"))
 (gr_arc (start 124.588016 92.241596) (mid 125.173799 90.827379) (end 126.588016 90.241596) (stroke (width 0.1) (type default))
  (layer "Edge.Cuts"))
 (gr_line (start 126.588016 90.241596) (end 162.070638 90.241596) (stroke (width 0.1) (type default)) (layer "Edge.Cuts"))
 (gr_arc (start 162.070638 90.241596) (mid 163.484843 90.827391) (end 164.070638 92.241596) (stroke (width 0.1) (type default))
  (layer "Edge.Cuts"))
 (gr_line (start 162.070638 109.652746) (end 126.588016 109.652746) (stroke (width 0.1) (type default)) (layer "Edge.Cuts"))
 (segment (start 140.777603 93.678459) (end 137.697184 93.678459) (width 0.5) (layer "F.Cu") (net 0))
 (segment (start 131.547175 93.645015) (end 128.330401 93.645015) (width 0.5) (layer "F.Cu") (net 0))
 (segment (start 156.189149 93.609236) (end 159.127427 93.609236) (width 0.5) (layer "F.Cu") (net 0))
 (segment (start 158.845254 106.353131) (end 158.889149 106.309236) (width 0.5) (layer "F.Cu") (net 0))
 (segment (start 156.189149 93.609236) (end 156.044675 93.75371) (width 0.5) (layer "F.Cu") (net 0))
 (segment (start 161.987212 106.347347) (end 158.92726 106.347347) (width 0.5) (layer "F.Cu") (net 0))
 (segment (start 162.287964 93.844773) (end 162.230345 93.787154) (width 0.5) (layer "F.Cu") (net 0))
 (segment (start 137.592182 93.645015) (end 137.627961 93.609236) (width 0.5) (layer "F.Cu") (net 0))
 (segment (start 146.984052 93.75371) (end 150.074917 93.75371) (width 0.5) (layer "F.Cu") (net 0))
 (segment (start 159.127427 93.609236) (end 159.305345 93.787154) (width 0.5) (layer "F.Cu") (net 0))
 (segment (start 128.330401 93.645015) (end 128.322285 93.653131) (width 0.5) (layer "F.Cu") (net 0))
 (segment (start 146.858145 93.678459) (end 146.883473 93.653131) (width 0.5) (layer "F.Cu") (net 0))
 (segment (start 134.472175 93.645015) (end 137.592182 93.645015) (width 0.5) (layer "F.Cu") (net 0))
 (segment (start 131.022285 106.353131) (end 158.845254 106.353131) (width 0.5) (layer "F.Cu") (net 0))
 (segment (start 143.702603 93.678459) (end 146.858145 93.678459) (width 0.5) (layer "F.Cu") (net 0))
 (segment (start 158.92726 106.347347) (end 158.889149 106.309236) (width 0.5) (layer "F.Cu") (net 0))
 (segment (start 162.287964 95.958051) (end 162.287964 93.844773) (width 0.5) (layer "F.Cu") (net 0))
 (segment (start 137.697184 93.678459) (end 137.627961 93.609236) (width 0.5) (layer "F.Cu") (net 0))
 (segment (start 146.883473 93.653131) (end 146.984052 93.75371) (width 0.5) (layer "F.Cu") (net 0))
 (segment (start 156.044675 93.75371) (end 152.999917 93.75371) (width 0.5) (layer "F.Cu") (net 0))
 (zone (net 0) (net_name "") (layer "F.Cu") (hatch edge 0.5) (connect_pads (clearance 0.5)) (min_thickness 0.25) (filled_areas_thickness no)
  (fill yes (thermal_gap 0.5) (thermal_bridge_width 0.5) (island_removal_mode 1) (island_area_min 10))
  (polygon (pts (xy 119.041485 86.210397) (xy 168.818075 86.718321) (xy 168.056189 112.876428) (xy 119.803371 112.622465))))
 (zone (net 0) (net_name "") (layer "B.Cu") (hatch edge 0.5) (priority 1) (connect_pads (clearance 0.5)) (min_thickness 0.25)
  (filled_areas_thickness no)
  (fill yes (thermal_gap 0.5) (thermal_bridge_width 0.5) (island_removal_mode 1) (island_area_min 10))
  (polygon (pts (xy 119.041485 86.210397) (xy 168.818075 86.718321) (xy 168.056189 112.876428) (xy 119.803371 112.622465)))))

